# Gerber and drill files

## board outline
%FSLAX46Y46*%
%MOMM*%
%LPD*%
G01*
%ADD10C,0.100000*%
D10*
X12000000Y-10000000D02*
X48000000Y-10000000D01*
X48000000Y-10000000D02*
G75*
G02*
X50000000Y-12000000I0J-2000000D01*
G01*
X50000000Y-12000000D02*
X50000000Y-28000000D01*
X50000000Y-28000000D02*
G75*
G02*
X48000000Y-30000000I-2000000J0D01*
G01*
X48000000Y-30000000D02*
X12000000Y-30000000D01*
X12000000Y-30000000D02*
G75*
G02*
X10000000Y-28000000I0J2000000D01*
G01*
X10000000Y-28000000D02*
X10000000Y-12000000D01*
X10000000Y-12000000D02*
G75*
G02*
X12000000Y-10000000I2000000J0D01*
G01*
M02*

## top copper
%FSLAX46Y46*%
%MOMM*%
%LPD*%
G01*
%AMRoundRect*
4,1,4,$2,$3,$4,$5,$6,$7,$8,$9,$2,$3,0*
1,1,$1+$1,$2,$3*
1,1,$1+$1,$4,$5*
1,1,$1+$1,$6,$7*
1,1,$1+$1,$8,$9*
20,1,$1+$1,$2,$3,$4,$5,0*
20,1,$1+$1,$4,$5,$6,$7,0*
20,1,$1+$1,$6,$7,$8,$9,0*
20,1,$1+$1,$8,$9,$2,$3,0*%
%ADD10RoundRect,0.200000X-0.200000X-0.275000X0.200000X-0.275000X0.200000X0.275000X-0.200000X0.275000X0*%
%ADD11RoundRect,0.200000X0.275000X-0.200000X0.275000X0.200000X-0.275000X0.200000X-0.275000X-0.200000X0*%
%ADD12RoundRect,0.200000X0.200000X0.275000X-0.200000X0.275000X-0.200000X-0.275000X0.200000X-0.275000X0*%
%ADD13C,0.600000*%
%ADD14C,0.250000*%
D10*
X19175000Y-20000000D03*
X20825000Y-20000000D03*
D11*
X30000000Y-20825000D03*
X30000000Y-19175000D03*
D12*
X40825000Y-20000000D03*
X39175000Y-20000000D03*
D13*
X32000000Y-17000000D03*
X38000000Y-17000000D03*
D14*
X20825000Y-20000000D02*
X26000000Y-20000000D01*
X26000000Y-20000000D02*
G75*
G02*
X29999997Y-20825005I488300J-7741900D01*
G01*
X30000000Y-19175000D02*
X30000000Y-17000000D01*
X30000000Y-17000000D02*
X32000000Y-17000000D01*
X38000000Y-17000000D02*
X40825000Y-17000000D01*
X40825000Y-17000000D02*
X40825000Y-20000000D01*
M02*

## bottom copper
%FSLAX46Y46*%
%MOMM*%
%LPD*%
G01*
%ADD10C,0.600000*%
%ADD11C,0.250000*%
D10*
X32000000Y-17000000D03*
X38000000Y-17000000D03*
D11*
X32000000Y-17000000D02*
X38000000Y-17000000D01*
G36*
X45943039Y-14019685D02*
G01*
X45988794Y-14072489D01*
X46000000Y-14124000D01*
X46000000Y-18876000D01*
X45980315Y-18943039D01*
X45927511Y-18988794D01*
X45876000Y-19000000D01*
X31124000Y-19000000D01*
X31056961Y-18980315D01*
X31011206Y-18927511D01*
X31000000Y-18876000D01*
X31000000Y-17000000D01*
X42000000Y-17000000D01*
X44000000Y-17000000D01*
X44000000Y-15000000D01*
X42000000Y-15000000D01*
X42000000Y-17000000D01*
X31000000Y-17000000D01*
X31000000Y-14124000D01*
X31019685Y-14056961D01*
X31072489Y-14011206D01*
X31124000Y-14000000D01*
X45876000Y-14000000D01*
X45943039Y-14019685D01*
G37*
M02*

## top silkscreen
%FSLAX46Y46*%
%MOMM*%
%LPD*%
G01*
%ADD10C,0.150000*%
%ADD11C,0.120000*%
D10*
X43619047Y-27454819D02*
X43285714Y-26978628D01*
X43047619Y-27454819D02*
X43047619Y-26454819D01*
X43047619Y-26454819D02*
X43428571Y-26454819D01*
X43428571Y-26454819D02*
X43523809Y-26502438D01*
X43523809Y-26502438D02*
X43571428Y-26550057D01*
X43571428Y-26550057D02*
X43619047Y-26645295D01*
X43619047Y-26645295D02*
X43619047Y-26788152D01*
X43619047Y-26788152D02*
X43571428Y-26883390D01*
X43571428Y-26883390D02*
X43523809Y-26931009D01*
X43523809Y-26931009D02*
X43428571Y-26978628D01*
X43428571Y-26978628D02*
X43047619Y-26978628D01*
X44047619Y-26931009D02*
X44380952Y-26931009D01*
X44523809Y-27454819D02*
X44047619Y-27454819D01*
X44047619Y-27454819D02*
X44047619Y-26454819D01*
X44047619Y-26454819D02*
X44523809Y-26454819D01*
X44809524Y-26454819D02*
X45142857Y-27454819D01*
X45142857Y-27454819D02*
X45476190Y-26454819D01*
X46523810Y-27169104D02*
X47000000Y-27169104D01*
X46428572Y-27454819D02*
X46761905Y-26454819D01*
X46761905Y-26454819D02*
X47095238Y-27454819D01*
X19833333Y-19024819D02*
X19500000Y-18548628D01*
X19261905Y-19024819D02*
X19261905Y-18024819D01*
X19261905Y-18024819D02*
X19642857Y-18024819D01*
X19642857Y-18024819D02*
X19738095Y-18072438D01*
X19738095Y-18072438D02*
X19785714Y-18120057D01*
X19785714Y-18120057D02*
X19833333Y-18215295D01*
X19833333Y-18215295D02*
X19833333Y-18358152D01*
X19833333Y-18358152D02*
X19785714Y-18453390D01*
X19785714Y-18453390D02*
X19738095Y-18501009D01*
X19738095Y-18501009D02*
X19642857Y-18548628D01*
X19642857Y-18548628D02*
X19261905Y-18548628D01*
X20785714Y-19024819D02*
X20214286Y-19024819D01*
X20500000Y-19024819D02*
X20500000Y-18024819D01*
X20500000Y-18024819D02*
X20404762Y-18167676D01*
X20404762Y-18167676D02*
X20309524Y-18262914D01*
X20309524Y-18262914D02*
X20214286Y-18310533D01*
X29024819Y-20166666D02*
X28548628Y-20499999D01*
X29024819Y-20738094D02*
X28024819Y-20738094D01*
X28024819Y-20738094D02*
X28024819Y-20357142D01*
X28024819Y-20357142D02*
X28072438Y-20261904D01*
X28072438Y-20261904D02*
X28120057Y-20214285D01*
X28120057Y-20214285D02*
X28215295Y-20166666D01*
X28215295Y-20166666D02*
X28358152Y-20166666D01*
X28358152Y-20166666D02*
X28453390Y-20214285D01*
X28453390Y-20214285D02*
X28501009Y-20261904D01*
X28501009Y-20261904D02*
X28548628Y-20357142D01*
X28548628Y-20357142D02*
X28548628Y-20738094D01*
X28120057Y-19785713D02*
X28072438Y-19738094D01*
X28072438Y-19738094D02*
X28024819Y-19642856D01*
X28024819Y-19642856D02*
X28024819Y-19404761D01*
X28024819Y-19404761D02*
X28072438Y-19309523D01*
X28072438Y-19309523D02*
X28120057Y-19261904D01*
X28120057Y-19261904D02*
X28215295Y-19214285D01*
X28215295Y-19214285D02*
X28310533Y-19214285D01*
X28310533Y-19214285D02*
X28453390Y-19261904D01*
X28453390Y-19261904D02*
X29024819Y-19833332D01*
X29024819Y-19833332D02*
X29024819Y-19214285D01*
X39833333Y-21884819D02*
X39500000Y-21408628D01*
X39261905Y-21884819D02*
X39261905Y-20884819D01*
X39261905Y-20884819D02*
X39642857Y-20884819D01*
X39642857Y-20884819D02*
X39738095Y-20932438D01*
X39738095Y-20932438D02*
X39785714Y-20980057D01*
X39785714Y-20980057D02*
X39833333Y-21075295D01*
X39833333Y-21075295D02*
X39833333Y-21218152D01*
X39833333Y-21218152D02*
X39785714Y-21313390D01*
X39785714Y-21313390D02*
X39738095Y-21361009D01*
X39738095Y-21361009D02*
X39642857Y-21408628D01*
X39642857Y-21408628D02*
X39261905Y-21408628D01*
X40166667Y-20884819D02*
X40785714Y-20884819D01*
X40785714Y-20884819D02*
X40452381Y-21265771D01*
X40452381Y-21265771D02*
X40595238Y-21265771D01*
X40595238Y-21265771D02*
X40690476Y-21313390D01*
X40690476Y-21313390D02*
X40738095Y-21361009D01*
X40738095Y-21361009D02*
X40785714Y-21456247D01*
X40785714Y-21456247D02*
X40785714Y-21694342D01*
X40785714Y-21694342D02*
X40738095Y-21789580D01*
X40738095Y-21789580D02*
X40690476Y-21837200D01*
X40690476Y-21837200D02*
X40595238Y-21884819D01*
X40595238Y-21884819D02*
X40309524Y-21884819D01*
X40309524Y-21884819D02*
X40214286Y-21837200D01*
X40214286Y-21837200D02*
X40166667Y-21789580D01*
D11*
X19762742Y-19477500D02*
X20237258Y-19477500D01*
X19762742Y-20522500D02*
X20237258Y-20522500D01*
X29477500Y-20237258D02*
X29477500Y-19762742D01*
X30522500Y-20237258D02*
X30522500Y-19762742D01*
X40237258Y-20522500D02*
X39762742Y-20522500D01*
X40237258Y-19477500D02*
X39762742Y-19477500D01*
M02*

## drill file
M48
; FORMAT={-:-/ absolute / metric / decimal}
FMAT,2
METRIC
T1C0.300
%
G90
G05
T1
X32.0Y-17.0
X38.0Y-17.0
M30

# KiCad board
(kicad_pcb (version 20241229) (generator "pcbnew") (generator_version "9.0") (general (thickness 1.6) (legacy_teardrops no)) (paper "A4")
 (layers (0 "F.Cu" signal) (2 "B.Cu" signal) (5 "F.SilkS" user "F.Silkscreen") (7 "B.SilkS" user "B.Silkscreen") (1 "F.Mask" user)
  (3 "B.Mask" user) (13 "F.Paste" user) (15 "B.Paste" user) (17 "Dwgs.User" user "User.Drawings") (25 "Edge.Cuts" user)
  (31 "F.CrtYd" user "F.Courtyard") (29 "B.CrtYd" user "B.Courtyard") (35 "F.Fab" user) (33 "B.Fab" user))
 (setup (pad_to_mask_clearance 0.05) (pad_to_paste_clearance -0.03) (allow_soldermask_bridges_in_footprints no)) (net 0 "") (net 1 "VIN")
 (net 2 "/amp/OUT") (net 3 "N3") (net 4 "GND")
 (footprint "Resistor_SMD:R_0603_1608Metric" (layer "F.Cu") (at 20 20)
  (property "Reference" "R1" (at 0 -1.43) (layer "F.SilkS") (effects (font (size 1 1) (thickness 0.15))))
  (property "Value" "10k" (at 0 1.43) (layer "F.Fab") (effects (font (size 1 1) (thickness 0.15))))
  (fp_line (start -0.237258 -0.5225) (end 0.237258 -0.5225) (stroke (width 0.12) (type solid)) (layer "F.SilkS"))
  (fp_line (start -0.237258 0.5225) (end 0.237258 0.5225) (stroke (width 0.12) (type solid)) (layer "F.SilkS"))
  (pad "1" smd roundrect (at -0.825 0) (size 0.8 0.95) (layers "F.Cu" "F.Mask" "F.Paste") (roundrect_rratio 0.25) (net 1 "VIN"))
  (pad "2" smd roundrect (at 0.825 0) (size 0.8 0.95) (layers "F.Cu" "F.Mask" "F.Paste") (roundrect_rratio 0.25) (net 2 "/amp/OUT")))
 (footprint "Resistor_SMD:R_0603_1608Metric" (layer "F.Cu") (at 30 20 90)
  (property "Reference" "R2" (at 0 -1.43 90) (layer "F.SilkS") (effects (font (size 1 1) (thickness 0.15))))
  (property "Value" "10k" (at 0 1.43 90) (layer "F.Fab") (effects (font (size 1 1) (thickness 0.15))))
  (fp_line (start -0.237258 -0.5225) (end 0.237258 -0.5225) (stroke (width 0.12) (type solid)) (layer "F.SilkS"))
  (fp_line (start -0.237258 0.5225) (end 0.237258 0.5225) (stroke (width 0.12) (type solid)) (layer "F.SilkS"))
  (pad "1" smd roundrect (at -0.825 0 90) (size 0.8 0.95) (layers "F.Cu" "F.Mask" "F.Paste") (roundrect_rratio 0.25) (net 2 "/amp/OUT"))
  (pad "2" smd roundrect (at 0.825 0 90) (size 0.8 0.95) (layers "F.Cu" "F.Mask" "F.Paste") (roundrect_rratio 0.25) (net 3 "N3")))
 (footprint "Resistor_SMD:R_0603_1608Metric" (layer "F.Cu") (at 40 20 180)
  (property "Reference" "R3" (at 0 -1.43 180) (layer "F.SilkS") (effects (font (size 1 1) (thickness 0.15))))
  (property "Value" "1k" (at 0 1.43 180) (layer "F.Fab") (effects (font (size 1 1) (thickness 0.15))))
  (fp_line (start -0.237258 -0.5225) (end 0.237258 -0.5225) (stroke (width 0.12) (type solid)) (layer "F.SilkS"))
  (fp_line (start -0.237258 0.5225) (end 0.237258 0.5225) (stroke (width 0.12) (type solid)) (layer "F.SilkS"))
  (pad "1" smd roundrect (at -0.825 0 180) (size 0.8 0.95) (layers "F.Cu" "F.Mask" "F.Paste") (roundrect_rratio 0.25) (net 3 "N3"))
  (pad "2" smd roundrect (at 0.825 0 180) (size 0.8 0.95) (layers "F.Cu" "F.Mask" "F.Paste") (roundrect_rratio 0.25) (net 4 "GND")))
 (segment (start 20.825 20) (end 26 20) (width 0.25) (layer "F.Cu") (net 2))
 (arc (start 26 20) (mid 28.5 20.25) (end 30 20.825) (width 0.25) (layer "F.Cu") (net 2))
 (segment (start 30 19.175) (end 30 17) (width 0.25) (layer "F.Cu") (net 3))
 (segment (start 30 17) (end 32 17) (width 0.25) (layer "F.Cu") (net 3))
 (via (at 32 17) (size 0.6) (drill 0.3) (layers "F.Cu" "B.Cu") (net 3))
 (segment (start 32 17) (end 38 17) (width 0.25) (layer "B.Cu") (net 3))
 (via (at 38 17) (size 0.6) (drill 0.3) (layers "F.Cu" "B.Cu") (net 3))
 (segment (start 38 17) (end 40.825 17) (width 0.25) (layer "F.Cu") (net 3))
 (segment (start 40.825 17) (end 40.825 20) (width 0.25) (layer "F.Cu") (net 3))
 (gr_line (start 12 10) (end 48 10) (stroke (width 0.1) (type default)) (layer "Edge.Cuts"))
 (gr_arc (start 48 10) (mid 49.414214 10.585786) (end 50 12) (stroke (width 0.1) (type default)) (layer "Edge.Cuts"))
 (gr_line (start 50 12) (end 50 28) (stroke (width 0.1) (type default)) (layer "Edge.Cuts"))
 (gr_arc (start 50 28) (mid 49.414214 29.414214) (end 48 30) (stroke (width 0.1) (type default)) (layer "Edge.Cuts"))
 (gr_line (start 48 30) (end 12 30) (stroke (width 0.1) (type default)) (layer "Edge.Cuts"))
 (gr_arc (start 12 30) (mid 10.585786 29.414214) (end 10 28) (stroke (width 0.1) (type default)) (layer "Edge.Cuts"))
 (gr_line (start 10 28) (end 10 12) (stroke (width 0.1) (type default)) (layer "Edge.Cuts"))
 (gr_arc (start 10 12) (mid 10.585786 10.585786) (end 12 10) (stroke (width 0.1) (type default)) (layer "Edge.Cuts"))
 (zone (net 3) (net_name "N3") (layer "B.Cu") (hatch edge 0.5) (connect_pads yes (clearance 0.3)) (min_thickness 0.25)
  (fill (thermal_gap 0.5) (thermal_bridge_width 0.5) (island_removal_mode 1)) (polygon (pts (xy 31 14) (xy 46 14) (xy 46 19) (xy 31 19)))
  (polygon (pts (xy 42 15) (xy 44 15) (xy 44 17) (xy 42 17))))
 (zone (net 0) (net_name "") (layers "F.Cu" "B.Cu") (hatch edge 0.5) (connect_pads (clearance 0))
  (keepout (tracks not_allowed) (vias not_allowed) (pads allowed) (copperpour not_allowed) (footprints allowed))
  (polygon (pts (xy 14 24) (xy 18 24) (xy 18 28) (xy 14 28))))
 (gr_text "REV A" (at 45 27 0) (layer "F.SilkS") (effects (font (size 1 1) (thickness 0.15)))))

